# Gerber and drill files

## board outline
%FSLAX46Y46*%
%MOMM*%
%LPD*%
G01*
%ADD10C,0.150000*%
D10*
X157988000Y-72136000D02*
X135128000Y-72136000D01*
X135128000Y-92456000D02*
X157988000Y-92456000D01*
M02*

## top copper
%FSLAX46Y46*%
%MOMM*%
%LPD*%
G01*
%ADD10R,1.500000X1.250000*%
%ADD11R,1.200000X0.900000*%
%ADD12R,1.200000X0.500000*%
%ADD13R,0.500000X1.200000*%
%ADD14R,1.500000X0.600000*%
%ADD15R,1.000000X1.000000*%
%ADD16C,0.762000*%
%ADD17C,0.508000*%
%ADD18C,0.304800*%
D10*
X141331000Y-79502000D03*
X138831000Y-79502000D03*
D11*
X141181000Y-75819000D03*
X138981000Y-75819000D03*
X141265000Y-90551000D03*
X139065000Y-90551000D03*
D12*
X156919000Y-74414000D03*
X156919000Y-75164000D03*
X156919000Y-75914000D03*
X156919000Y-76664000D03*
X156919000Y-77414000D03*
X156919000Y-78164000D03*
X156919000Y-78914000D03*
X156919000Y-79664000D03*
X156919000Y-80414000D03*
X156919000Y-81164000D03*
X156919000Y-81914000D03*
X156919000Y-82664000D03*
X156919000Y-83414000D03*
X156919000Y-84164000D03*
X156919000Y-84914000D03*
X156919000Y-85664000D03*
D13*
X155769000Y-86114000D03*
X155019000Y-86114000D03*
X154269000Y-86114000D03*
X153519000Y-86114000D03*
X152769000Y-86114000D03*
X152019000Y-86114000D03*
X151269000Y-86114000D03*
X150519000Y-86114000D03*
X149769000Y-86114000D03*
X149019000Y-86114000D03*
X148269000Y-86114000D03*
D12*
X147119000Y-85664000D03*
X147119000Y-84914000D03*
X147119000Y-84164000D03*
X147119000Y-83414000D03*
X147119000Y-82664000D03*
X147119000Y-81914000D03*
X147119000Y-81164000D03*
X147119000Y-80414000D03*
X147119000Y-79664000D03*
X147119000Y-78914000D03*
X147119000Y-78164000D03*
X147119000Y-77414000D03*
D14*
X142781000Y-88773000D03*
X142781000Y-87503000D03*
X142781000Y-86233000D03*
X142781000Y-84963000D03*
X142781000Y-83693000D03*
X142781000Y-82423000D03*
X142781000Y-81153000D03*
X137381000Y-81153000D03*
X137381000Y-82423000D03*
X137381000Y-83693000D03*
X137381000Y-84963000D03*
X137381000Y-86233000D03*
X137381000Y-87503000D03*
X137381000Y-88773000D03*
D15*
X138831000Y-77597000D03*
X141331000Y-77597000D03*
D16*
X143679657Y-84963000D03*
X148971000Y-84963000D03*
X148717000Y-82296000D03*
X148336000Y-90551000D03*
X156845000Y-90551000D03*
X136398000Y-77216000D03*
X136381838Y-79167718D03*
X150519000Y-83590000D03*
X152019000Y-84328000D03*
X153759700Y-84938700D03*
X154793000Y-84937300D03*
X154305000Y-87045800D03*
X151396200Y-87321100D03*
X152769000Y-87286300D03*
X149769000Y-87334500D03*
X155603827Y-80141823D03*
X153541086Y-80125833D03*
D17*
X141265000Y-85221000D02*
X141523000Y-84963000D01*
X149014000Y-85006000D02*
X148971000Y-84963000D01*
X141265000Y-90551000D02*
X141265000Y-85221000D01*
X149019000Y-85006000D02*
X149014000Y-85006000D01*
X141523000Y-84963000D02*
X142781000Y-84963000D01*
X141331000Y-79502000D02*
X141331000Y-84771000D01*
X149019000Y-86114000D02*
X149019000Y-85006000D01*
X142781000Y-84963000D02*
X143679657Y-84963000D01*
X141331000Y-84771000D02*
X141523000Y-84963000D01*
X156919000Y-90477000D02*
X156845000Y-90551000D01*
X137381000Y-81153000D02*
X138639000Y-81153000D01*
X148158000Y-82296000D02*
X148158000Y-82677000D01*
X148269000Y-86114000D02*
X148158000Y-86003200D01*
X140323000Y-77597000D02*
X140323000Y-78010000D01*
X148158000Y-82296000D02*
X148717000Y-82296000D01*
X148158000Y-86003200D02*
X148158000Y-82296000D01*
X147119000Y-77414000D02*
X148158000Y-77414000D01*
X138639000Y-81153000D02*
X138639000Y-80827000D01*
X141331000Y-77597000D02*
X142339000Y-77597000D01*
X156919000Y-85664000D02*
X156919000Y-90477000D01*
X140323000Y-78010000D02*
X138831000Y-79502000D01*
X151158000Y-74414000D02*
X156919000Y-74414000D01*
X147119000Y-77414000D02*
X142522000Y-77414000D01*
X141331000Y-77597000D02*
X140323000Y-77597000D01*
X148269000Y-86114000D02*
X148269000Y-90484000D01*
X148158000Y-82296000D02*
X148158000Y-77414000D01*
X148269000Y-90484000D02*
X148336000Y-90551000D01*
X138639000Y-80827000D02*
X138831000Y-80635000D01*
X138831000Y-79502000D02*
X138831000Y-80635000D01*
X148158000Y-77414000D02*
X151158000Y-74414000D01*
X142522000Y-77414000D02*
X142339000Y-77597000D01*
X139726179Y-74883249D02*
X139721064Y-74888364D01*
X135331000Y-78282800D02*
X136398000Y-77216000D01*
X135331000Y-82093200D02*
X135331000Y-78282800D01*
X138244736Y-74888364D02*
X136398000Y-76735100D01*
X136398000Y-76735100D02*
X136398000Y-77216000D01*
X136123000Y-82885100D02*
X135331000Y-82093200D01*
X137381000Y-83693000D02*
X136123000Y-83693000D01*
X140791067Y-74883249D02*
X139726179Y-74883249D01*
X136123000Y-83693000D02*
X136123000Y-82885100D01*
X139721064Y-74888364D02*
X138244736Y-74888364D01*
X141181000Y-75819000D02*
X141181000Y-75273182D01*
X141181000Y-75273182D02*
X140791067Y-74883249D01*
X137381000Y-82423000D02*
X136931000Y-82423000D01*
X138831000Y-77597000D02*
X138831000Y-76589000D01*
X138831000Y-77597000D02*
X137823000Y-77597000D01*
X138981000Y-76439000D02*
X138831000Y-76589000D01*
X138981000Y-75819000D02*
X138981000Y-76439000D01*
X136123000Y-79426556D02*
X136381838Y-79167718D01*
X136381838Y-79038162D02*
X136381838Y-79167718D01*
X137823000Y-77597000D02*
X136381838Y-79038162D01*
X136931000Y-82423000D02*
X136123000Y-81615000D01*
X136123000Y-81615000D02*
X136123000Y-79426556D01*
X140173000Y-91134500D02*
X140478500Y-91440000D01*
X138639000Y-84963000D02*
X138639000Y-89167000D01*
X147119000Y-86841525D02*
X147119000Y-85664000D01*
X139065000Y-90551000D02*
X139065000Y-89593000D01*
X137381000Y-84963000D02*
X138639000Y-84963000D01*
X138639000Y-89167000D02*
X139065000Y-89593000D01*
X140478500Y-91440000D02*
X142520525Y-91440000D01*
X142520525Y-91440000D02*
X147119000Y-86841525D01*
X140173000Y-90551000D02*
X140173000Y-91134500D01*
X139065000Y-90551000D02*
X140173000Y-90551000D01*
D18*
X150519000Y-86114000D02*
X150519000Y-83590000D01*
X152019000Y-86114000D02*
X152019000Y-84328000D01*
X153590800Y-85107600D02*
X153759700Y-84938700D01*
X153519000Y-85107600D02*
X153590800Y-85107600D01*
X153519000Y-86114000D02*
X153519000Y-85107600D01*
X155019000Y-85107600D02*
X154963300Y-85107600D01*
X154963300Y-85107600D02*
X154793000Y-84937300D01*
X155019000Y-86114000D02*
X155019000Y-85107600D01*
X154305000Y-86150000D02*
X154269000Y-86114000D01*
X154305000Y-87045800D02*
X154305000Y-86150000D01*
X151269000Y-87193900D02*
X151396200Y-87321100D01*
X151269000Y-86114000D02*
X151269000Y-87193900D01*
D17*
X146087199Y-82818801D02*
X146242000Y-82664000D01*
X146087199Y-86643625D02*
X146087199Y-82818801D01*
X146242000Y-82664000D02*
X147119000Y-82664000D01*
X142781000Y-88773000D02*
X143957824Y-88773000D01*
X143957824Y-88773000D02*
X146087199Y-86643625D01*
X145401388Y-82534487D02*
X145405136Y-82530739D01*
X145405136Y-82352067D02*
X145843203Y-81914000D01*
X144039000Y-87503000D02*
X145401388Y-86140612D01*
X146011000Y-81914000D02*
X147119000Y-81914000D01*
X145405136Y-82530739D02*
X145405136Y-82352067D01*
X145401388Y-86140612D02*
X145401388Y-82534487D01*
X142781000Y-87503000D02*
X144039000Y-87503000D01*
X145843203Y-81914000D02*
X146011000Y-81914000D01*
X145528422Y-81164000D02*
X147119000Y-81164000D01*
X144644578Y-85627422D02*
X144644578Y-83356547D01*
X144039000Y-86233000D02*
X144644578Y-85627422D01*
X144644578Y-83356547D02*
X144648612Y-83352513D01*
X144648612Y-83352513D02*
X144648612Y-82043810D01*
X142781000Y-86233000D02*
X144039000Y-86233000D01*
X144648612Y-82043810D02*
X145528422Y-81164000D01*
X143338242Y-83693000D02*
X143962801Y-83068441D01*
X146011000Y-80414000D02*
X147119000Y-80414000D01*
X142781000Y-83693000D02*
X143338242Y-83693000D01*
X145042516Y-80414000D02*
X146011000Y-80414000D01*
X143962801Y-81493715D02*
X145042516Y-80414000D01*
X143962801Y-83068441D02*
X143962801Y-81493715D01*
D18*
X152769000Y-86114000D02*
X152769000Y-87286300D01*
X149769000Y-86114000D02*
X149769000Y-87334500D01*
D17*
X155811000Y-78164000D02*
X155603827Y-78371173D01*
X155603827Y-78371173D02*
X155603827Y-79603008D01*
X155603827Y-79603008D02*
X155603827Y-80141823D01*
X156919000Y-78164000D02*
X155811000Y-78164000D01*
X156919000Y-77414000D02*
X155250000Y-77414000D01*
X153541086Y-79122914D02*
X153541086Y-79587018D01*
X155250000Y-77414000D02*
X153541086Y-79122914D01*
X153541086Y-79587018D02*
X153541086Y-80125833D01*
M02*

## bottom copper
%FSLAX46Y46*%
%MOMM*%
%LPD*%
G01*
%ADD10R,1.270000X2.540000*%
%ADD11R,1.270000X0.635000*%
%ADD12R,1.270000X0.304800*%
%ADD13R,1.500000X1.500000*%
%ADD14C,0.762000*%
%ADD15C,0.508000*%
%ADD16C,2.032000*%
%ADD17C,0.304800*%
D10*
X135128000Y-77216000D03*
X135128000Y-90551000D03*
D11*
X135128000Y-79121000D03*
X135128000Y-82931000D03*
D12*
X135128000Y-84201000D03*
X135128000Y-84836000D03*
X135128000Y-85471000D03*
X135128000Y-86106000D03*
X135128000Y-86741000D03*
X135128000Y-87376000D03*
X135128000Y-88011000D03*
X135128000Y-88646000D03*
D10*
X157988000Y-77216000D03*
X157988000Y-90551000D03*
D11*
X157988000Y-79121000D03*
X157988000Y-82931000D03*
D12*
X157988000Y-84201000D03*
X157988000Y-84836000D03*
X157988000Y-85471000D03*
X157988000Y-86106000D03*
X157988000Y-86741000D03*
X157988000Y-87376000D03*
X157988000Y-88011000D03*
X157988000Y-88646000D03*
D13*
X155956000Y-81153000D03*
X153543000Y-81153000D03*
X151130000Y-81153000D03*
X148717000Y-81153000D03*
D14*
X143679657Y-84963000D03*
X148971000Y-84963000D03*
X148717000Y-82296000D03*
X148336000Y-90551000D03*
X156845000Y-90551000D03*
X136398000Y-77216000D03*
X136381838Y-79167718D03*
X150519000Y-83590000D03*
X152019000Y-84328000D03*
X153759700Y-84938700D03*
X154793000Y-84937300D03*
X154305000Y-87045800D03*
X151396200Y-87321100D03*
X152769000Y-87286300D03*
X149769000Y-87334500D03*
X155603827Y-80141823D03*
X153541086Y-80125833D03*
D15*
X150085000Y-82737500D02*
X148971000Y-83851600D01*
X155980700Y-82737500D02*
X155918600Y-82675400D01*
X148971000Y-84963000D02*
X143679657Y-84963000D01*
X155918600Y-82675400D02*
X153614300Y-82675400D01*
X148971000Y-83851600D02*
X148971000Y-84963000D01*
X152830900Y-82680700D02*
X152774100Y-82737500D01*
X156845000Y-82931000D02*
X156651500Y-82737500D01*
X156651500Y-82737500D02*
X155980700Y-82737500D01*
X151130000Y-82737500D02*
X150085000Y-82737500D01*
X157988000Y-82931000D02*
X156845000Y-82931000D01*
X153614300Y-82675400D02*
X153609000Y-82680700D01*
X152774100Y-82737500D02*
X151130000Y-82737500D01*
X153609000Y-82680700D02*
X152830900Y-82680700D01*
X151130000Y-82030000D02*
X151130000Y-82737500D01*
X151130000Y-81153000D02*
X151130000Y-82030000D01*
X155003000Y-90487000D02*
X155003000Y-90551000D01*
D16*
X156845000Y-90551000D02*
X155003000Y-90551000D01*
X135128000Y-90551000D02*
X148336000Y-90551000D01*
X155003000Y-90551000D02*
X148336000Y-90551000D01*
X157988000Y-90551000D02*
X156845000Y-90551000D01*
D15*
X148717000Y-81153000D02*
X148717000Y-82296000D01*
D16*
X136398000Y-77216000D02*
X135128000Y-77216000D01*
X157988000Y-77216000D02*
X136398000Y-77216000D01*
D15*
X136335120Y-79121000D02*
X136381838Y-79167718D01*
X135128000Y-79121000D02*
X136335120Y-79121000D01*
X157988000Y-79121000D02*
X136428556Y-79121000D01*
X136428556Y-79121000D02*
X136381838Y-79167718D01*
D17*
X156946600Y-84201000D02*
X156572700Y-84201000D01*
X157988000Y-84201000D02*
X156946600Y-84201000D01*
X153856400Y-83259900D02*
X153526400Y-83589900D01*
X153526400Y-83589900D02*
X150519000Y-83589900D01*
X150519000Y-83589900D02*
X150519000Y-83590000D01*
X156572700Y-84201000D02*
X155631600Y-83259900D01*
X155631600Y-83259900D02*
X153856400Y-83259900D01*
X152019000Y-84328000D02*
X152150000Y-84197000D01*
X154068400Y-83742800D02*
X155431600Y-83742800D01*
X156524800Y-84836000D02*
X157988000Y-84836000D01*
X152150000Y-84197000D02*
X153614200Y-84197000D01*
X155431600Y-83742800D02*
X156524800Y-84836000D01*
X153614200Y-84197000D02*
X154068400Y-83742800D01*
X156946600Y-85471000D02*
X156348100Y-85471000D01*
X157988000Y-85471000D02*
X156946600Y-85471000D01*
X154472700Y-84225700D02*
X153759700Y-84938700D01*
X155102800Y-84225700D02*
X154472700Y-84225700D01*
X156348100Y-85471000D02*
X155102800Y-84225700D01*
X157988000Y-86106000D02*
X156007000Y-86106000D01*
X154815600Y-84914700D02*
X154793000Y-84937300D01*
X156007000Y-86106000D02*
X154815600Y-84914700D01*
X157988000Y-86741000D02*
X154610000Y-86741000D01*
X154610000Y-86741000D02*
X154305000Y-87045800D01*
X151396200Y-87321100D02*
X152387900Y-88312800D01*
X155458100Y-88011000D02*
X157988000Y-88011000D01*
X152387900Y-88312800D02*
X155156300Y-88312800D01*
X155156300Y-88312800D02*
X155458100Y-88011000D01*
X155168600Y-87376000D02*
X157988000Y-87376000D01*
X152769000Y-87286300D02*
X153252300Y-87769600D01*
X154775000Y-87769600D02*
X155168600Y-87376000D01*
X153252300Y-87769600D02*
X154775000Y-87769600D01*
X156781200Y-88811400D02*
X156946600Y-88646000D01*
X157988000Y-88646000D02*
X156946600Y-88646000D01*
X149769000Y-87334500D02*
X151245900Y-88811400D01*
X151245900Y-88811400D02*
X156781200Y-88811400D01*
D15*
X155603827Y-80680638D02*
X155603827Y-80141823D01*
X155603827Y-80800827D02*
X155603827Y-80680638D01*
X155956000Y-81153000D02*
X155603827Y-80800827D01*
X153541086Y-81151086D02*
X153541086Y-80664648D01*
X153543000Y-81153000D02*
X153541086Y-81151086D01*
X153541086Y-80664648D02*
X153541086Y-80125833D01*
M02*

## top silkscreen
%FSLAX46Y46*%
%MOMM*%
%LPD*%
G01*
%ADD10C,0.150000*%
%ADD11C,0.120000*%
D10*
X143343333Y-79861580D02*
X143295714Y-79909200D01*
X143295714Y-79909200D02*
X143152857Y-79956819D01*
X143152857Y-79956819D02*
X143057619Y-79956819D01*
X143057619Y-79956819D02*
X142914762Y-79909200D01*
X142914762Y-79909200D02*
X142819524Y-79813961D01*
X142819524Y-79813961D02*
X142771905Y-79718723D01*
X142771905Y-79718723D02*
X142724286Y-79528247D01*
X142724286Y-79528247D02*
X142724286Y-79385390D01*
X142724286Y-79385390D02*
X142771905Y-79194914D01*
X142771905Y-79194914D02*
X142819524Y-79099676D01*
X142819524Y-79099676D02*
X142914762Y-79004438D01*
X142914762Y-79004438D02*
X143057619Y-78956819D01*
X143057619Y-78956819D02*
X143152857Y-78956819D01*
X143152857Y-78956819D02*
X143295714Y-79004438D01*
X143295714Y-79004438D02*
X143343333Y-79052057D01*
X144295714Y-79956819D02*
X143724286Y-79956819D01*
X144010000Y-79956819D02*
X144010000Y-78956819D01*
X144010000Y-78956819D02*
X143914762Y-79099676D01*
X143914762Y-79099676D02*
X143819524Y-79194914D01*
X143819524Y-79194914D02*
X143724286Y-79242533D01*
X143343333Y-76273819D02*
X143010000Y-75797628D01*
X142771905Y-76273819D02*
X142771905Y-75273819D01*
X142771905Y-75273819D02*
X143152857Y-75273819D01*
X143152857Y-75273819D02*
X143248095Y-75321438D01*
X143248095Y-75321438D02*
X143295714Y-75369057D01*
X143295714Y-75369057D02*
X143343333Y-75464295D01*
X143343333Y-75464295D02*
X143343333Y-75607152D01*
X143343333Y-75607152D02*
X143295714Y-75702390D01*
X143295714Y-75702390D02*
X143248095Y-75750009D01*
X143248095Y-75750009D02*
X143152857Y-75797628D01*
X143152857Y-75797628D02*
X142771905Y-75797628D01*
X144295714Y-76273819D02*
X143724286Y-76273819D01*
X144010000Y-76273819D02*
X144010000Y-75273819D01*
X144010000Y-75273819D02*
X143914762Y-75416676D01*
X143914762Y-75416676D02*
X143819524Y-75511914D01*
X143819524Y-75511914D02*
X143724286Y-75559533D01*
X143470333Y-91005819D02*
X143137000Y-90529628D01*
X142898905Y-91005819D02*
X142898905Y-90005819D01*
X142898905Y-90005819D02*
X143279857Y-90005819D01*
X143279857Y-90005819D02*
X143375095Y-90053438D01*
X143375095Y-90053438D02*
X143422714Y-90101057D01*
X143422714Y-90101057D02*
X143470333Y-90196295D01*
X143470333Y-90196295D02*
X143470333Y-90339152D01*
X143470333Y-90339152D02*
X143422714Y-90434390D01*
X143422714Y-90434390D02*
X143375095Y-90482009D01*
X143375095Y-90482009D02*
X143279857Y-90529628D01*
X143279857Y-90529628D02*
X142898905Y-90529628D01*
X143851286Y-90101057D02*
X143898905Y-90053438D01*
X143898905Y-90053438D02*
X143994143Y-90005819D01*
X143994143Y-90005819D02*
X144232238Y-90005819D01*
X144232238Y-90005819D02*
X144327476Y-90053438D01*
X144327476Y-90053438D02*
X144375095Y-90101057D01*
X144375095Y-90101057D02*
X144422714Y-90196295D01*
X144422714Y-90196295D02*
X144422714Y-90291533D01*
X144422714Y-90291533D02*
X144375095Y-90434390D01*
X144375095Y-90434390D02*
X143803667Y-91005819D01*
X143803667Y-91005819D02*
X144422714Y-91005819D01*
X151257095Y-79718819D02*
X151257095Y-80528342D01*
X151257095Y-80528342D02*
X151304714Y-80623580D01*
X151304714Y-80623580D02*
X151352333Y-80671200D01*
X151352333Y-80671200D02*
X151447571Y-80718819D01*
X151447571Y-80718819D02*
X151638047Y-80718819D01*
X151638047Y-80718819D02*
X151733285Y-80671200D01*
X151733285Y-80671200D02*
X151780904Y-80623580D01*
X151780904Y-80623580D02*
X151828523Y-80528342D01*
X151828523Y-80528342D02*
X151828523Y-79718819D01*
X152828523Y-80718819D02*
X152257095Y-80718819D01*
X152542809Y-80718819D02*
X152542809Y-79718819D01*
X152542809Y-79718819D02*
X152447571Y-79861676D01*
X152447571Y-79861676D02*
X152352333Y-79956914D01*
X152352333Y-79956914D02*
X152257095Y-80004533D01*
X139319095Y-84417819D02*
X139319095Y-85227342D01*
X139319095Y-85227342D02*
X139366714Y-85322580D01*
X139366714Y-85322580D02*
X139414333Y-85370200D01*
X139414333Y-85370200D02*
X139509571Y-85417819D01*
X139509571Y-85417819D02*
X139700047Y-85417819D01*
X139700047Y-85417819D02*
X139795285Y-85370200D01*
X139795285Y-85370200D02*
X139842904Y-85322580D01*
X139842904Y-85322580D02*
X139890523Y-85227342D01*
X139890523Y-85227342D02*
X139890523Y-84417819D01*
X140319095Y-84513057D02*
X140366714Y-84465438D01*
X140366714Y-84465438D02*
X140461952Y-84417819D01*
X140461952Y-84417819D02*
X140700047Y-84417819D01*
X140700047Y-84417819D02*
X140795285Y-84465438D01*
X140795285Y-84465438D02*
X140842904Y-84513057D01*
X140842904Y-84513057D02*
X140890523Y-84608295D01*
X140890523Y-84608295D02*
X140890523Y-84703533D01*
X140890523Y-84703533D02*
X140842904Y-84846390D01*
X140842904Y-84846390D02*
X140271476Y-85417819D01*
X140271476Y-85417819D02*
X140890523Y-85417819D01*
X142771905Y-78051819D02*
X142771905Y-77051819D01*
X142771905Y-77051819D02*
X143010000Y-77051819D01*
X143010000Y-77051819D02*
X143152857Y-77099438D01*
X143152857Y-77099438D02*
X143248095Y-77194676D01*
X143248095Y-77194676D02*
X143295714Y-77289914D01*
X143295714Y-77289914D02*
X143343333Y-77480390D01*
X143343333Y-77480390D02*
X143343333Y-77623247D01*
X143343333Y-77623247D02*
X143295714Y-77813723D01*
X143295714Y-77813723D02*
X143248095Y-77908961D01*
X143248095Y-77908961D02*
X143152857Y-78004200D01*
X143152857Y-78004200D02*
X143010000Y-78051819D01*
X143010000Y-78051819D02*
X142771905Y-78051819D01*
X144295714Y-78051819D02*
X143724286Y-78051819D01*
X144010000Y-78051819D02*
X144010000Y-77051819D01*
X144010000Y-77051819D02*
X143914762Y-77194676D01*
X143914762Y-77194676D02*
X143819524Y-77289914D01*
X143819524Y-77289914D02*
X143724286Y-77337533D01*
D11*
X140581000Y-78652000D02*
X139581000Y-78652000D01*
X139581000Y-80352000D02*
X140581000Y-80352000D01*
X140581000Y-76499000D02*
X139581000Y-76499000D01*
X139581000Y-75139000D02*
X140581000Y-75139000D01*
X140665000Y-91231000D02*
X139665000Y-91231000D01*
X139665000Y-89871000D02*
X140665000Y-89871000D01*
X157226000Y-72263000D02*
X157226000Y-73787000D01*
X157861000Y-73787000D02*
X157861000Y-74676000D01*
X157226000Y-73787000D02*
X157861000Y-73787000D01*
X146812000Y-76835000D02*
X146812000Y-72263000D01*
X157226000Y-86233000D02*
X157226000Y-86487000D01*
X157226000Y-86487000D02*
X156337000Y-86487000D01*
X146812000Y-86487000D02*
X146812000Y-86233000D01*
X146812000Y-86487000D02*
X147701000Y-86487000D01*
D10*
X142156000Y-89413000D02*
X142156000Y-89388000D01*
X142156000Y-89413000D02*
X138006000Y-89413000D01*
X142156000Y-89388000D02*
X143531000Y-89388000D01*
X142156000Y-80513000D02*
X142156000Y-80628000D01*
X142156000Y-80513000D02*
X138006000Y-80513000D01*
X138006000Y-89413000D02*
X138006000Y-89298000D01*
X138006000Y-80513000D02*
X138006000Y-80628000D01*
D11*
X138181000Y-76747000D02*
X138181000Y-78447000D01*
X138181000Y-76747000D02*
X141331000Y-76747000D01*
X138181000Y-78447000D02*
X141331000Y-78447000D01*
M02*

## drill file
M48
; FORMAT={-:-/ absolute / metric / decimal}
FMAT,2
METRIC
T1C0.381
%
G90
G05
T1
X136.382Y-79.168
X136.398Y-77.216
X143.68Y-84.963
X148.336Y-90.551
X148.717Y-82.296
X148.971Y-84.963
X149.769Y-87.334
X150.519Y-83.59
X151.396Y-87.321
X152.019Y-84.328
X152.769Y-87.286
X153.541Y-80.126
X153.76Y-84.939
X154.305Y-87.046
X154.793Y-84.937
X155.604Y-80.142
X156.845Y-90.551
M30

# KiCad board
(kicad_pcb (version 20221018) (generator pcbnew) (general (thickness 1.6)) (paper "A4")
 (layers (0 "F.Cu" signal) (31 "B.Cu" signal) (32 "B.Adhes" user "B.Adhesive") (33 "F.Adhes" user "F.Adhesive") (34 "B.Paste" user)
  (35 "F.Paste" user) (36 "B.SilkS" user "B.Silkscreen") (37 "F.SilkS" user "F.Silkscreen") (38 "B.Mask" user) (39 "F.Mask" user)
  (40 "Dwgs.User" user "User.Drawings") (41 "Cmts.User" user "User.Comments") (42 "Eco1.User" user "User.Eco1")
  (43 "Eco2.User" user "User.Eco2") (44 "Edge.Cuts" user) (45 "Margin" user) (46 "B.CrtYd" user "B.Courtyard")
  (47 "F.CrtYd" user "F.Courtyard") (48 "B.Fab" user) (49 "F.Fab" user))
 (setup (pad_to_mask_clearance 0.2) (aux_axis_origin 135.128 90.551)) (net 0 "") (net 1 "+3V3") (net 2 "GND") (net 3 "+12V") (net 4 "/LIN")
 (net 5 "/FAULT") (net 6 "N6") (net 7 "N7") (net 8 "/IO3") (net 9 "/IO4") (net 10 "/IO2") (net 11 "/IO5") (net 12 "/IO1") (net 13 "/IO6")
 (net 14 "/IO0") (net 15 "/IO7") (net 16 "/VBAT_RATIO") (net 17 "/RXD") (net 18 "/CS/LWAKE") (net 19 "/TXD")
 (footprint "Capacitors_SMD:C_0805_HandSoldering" (layer "F.Cu") (at 140.081 79.502 180)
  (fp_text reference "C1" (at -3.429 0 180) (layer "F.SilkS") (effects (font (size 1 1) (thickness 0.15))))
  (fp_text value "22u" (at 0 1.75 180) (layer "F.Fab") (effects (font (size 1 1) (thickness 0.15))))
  (fp_line (start -0.5 0.85) (end 0.5 0.85) (stroke (width 0.12) (type solid)) (layer "F.SilkS"))
  (fp_line (start 0.5 -0.85) (end -0.5 -0.85) (stroke (width 0.12) (type solid)) (layer "F.SilkS"))
  (pad "1" smd rect (at -1.25 0 180) (size 1.5 1.25) (layers "F.Cu" "F.Paste" "F.Mask") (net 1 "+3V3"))
  (pad "2" smd rect (at 1.25 0 180) (size 1.5 1.25) (layers "F.Cu" "F.Paste" "F.Mask") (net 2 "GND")))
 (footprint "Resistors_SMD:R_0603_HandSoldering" (layer "F.Cu") (at 140.081 75.819 180)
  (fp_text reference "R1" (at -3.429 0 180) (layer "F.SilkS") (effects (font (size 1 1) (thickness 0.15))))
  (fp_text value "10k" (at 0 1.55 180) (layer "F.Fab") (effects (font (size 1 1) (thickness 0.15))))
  (fp_line (start -0.5 -0.68) (end 0.5 -0.68) (stroke (width 0.12) (type solid)) (layer "F.SilkS"))
  (fp_line (start 0.5 0.68) (end -0.5 0.68) (stroke (width 0.12) (type solid)) (layer "F.SilkS"))
  (pad "1" smd rect (at -1.1 0 180) (size 1.2 0.9) (layers "F.Cu" "F.Paste" "F.Mask") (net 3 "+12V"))
  (pad "2" smd rect (at 1.1 0 180) (size 1.2 0.9) (layers "F.Cu" "F.Paste" "F.Mask") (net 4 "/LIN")))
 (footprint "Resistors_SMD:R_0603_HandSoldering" (layer "F.Cu") (at 140.165 90.551 180)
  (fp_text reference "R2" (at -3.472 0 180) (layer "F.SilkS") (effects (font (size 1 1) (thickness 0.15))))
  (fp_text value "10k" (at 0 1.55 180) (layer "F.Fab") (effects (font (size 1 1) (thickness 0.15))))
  (fp_line (start -0.5 -0.68) (end 0.5 -0.68) (stroke (width 0.12) (type solid)) (layer "F.SilkS"))
  (fp_line (start 0.5 0.68) (end -0.5 0.68) (stroke (width 0.12) (type solid)) (layer "F.SilkS"))
  (pad "1" smd rect (at -1.1 0 180) (size 1.2 0.9) (layers "F.Cu" "F.Paste" "F.Mask") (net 1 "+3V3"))
  (pad "2" smd rect (at 1.1 0 180) (size 1.2 0.9) (layers "F.Cu" "F.Paste" "F.Mask") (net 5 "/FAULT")))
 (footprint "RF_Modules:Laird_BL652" (layer "F.Cu") (at 152.019 80.264 -90)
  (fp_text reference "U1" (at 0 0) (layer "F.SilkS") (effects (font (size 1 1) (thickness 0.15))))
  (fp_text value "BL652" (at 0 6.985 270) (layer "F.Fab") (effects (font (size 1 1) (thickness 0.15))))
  (fp_line (start -8.001 -5.207) (end -6.477 -5.207) (stroke (width 0.12) (type solid)) (layer "F.SilkS"))
  (fp_line (start -6.477 -5.842) (end -5.588 -5.842) (stroke (width 0.12) (type solid)) (layer "F.SilkS"))
  (fp_line (start -6.477 -5.207) (end -6.477 -5.842) (stroke (width 0.12) (type solid)) (layer "F.SilkS"))
  (fp_line (start -3.429 5.207) (end -8.001 5.207) (stroke (width 0.12) (type solid)) (layer "F.SilkS"))
  (fp_line (start 5.969 -5.207) (end 6.223 -5.207) (stroke (width 0.12) (type solid)) (layer "F.SilkS"))
  (fp_line (start 6.223 -5.207) (end 6.223 -4.318) (stroke (width 0.12) (type solid)) (layer "F.SilkS"))
  (fp_line (start 6.223 5.207) (end 5.969 5.207) (stroke (width 0.12) (type solid)) (layer "F.SilkS"))
  (fp_line (start 6.223 5.207) (end 6.223 4.318) (stroke (width 0.12) (type solid)) (layer "F.SilkS"))
  (pad "1" smd rect (at -5.85 -4.9) (size 1.2 0.5) (layers "F.Cu" "F.Paste" "F.Mask") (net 2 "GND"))
  (pad "2" smd rect (at -5.1 -4.9) (size 1.2 0.5) (layers "F.Cu" "F.Paste" "F.Mask"))
  (pad "3" smd rect (at -4.35 -4.9) (size 1.2 0.5) (layers "F.Cu" "F.Paste" "F.Mask"))
  (pad "4" smd rect (at -3.6 -4.9) (size 1.2 0.5) (layers "F.Cu" "F.Paste" "F.Mask"))
  (pad "5" smd rect (at -2.85 -4.9) (size 1.2 0.5) (layers "F.Cu" "F.Paste" "F.Mask") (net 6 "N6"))
  (pad "6" smd rect (at -2.1 -4.9) (size 1.2 0.5) (layers "F.Cu" "F.Paste" "F.Mask") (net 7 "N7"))
  (pad "7" smd rect (at -1.35 -4.9) (size 1.2 0.5) (layers "F.Cu" "F.Paste" "F.Mask"))
  (pad "8" smd rect (at -0.6 -4.9) (size 1.2 0.5) (layers "F.Cu" "F.Paste" "F.Mask"))
  (pad "9" smd rect (at 0.15 -4.9) (size 1.2 0.5) (layers "F.Cu" "F.Paste" "F.Mask"))
  (pad "10" smd rect (at 0.9 -4.9) (size 1.2 0.5) (layers "F.Cu" "F.Paste" "F.Mask"))
  (pad "11" smd rect (at 1.65 -4.9) (size 1.2 0.5) (layers "F.Cu" "F.Paste" "F.Mask"))
  (pad "12" smd rect (at 2.4 -4.9) (size 1.2 0.5) (layers "F.Cu" "F.Paste" "F.Mask"))
  (pad "13" smd rect (at 3.15 -4.9) (size 1.2 0.5) (layers "F.Cu" "F.Paste" "F.Mask"))
  (pad "14" smd rect (at 3.9 -4.9) (size 1.2 0.5) (layers "F.Cu" "F.Paste" "F.Mask"))
  (pad "15" smd rect (at 4.65 -4.9) (size 1.2 0.5) (layers "F.Cu" "F.Paste" "F.Mask"))
  (pad "16" smd rect (at 5.4 -4.9) (size 1.2 0.5) (layers "F.Cu" "F.Paste" "F.Mask") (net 2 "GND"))
  (pad "17" smd rect (at 5.85 -3.75 270) (size 1.2 0.5) (layers "F.Cu" "F.Paste" "F.Mask"))
  (pad "18" smd rect (at 5.85 -3 270) (size 1.2 0.5) (layers "F.Cu" "F.Paste" "F.Mask") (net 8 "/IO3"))
  (pad "19" smd rect (at 5.85 -2.25 270) (size 1.2 0.5) (layers "F.Cu" "F.Paste" "F.Mask") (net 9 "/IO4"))
  (pad "20" smd rect (at 5.85 -1.5 270) (size 1.2 0.5) (layers "F.Cu" "F.Paste" "F.Mask") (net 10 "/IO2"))
  (pad "21" smd rect (at 5.85 -0.75 270) (size 1.2 0.5) (layers "F.Cu" "F.Paste" "F.Mask") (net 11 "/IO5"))
  (pad "22" smd rect (at 5.85 0 270) (size 1.2 0.5) (layers "F.Cu" "F.Paste" "F.Mask") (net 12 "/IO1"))
  (pad "23" smd rect (at 5.85 0.75 270) (size 1.2 0.5) (layers "F.Cu" "F.Paste" "F.Mask") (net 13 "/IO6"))
  (pad "24" smd rect (at 5.85 1.5 270) (size 1.2 0.5) (layers "F.Cu" "F.Paste" "F.Mask") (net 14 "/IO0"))
  (pad "25" smd rect (at 5.85 2.25 270) (size 1.2 0.5) (layers "F.Cu" "F.Paste" "F.Mask") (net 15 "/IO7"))
  (pad "26" smd rect (at 5.85 3 270) (size 1.2 0.5) (layers "F.Cu" "F.Paste" "F.Mask") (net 1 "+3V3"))
  (pad "27" smd rect (at 5.85 3.75 270) (size 1.2 0.5) (layers "F.Cu" "F.Paste" "F.Mask") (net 2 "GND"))
  (pad "28" smd rect (at 5.4 4.9) (size 1.2 0.5) (layers "F.Cu" "F.Paste" "F.Mask") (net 5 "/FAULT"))
  (pad "29" smd rect (at 4.65 4.9) (size 1.2 0.5) (layers "F.Cu" "F.Paste" "F.Mask"))
  (pad "30" smd rect (at 3.9 4.9) (size 1.2 0.5) (layers "F.Cu" "F.Paste" "F.Mask"))
  (pad "31" smd rect (at 3.15 4.9) (size 1.2 0.5) (layers "F.Cu" "F.Paste" "F.Mask"))
  (pad "32" smd rect (at 2.4 4.9) (size 1.2 0.5) (layers "F.Cu" "F.Paste" "F.Mask") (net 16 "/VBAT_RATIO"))
  (pad "33" smd rect (at 1.65 4.9) (size 1.2 0.5) (layers "F.Cu" "F.Paste" "F.Mask") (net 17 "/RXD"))
  (pad "34" smd rect (at 0.9 4.9) (size 1.2 0.5) (layers "F.Cu" "F.Paste" "F.Mask") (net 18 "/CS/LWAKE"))
  (pad "35" smd rect (at 0.15 4.9) (size 1.2 0.5) (layers "F.Cu" "F.Paste" "F.Mask") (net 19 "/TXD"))
  (pad "36" smd rect (at -0.6 4.9) (size 1.2 0.5) (layers "F.Cu" "F.Paste" "F.Mask"))
  (pad "37" smd rect (at -1.35 4.9) (size 1.2 0.5) (layers "F.Cu" "F.Paste" "F.Mask"))
  (pad "38" smd rect (at -2.1 4.9) (size 1.2 0.5) (layers "F.Cu" "F.Paste" "F.Mask"))
  (pad "39" smd rect (at -2.85 4.9) (size 1.2 0.5) (layers "F.Cu" "F.Paste" "F.Mask") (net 2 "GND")))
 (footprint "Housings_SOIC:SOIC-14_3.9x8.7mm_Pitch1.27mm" (layer "F.Cu") (at 140.081 84.963 180)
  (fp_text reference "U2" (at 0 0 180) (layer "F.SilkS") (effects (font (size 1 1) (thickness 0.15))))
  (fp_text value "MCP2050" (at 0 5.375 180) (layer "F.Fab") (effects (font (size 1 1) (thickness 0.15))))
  (fp_line (start -2.075 -4.45) (end -2.075 -4.425) (stroke (width 0.15) (type solid)) (layer "F.SilkS"))
  (fp_line (start -2.075 -4.45) (end 2.075 -4.45) (stroke (width 0.15) (type solid)) (layer "F.SilkS"))
  (fp_line (start -2.075 -4.425) (end -3.45 -4.425) (stroke (width 0.15) (type solid)) (layer "F.SilkS"))
  (fp_line (start -2.075 4.45) (end -2.075 4.335) (stroke (width 0.15) (type solid)) (layer "F.SilkS"))
  (fp_line (start -2.075 4.45) (end 2.075 4.45) (stroke (width 0.15) (type solid)) (layer "F.SilkS"))
  (fp_line (start 2.075 -4.45) (end 2.075 -4.335) (stroke (width 0.15) (type solid)) (layer "F.SilkS"))
  (fp_line (start 2.075 4.45) (end 2.075 4.335) (stroke (width 0.15) (type solid)) (layer "F.SilkS"))
  (pad "1" smd rect (at -2.7 -3.81 180) (size 1.5 0.6) (layers "F.Cu" "F.Paste" "F.Mask") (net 16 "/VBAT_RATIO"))
  (pad "2" smd rect (at -2.7 -2.54 180) (size 1.5 0.6) (layers "F.Cu" "F.Paste" "F.Mask") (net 17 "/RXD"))
  (pad "3" smd rect (at -2.7 -1.27 180) (size 1.5 0.6) (layers "F.Cu" "F.Paste" "F.Mask") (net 18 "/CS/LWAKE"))
  (pad "4" smd rect (at -2.7 0 180) (size 1.5 0.6) (layers "F.Cu" "F.Paste" "F.Mask") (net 1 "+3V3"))
  (pad "5" smd rect (at -2.7 1.27 180) (size 1.5 0.6) (layers "F.Cu" "F.Paste" "F.Mask") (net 19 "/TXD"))
  (pad "6" smd rect (at -2.7 2.54 180) (size 1.5 0.6) (layers "F.Cu" "F.Paste" "F.Mask"))
  (pad "7" smd rect (at -2.7 3.81 180) (size 1.5 0.6) (layers "F.Cu" "F.Paste" "F.Mask"))
  (pad "8" smd rect (at 2.7 3.81 180) (size 1.5 0.6) (layers "F.Cu" "F.Paste" "F.Mask") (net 2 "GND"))
  (pad "9" smd rect (at 2.7 2.54 180) (size 1.5 0.6) (layers "F.Cu" "F.Paste" "F.Mask") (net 4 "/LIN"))
  (pad "10" smd rect (at 2.7 1.27 180) (size 1.5 0.6) (layers "F.Cu" "F.Paste" "F.Mask") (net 3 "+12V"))
  (pad "11" smd rect (at 2.7 0 180) (size 1.5 0.6) (layers "F.Cu" "F.Paste" "F.Mask") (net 5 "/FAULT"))
  (pad "12" smd rect (at 2.7 -1.27 180) (size 1.5 0.6) (layers "F.Cu" "F.Paste" "F.Mask"))
  (pad "13" smd rect (at 2.7 -2.54 180) (size 1.5 0.6) (layers "F.Cu" "F.Paste" "F.Mask"))
  (pad "14" smd rect (at 2.7 -3.81 180) (size 1.5 0.6) (layers "F.Cu" "F.Paste" "F.Mask")))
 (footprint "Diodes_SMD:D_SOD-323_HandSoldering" (layer "F.Cu") (at 140.081 77.597)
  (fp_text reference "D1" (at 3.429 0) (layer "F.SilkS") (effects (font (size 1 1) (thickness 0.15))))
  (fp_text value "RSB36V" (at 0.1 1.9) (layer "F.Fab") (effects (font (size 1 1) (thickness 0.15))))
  (fp_line (start -1.9 -0.85) (end -1.9 0.85) (stroke (width 0.12) (type solid)) (layer "F.SilkS"))
  (fp_line (start -1.9 -0.85) (end 1.25 -0.85) (stroke (width 0.12) (type solid)) (layer "F.SilkS"))
  (fp_line (start -1.9 0.85) (end 1.25 0.85) (stroke (width 0.12) (type solid)) (layer "F.SilkS"))
  (pad "1" smd rect (at -1.25 0) (size 1 1) (layers "F.Cu" "F.Paste" "F.Mask") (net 4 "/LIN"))
  (pad "2" smd rect (at 1.25 0) (size 1 1) (layers "F.Cu" "F.Paste" "F.Mask") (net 2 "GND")))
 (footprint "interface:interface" (layer "F.Cu") (at 135.128 72.771)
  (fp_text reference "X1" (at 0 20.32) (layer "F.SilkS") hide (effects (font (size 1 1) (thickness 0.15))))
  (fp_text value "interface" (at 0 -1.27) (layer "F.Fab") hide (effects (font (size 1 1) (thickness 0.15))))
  (pad "1" smd rect (at 0 4.445) (size 1.27 2.54) (layers "B.Cu") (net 3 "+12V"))
  (pad "2" smd rect (at 0 17.78) (size 1.27 2.54) (layers "B.Cu") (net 2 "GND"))
  (pad "3" smd rect (at 0 6.35) (size 1.27 0.635) (layers "B.Cu") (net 4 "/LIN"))
  (pad "4" smd rect (at 0 10.16) (size 1.27 0.635) (layers "B.Cu"))
  (pad "5" smd rect (at 0 11.43) (size 1.27 0.3048) (layers "B.Cu"))
  (pad "6" smd rect (at 0 12.065) (size 1.27 0.3048) (layers "B.Cu"))
  (pad "7" smd rect (at 0 12.7) (size 1.27 0.3048) (layers "B.Cu"))
  (pad "8" smd rect (at 0 13.335) (size 1.27 0.3048) (layers "B.Cu"))
  (pad "9" smd rect (at 0 13.97) (size 1.27 0.3048) (layers "B.Cu"))
  (pad "10" smd rect (at 0 14.605) (size 1.27 0.3048) (layers "B.Cu"))
  (pad "11" smd rect (at 0 15.24) (size 1.27 0.3048) (layers "B.Cu"))
  (pad "12" smd rect (at 0 15.875) (size 1.27 0.3048) (layers "B.Cu")))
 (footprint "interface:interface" (layer "F.Cu") (at 157.988 72.771)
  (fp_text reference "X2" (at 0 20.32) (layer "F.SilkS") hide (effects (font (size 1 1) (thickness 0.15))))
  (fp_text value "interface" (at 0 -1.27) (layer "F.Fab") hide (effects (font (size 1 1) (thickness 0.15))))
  (pad "1" smd rect (at 0 4.445) (size 1.27 2.54) (layers "B.Cu") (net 3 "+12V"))
  (pad "2" smd rect (at 0 17.78) (size 1.27 2.54) (layers "B.Cu") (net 2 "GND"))
  (pad "3" smd rect (at 0 6.35) (size 1.27 0.635) (layers "B.Cu") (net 4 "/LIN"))
  (pad "4" smd rect (at 0 10.16) (size 1.27 0.635) (layers "B.Cu") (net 1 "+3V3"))
  (pad "5" smd rect (at 0 11.43) (size 1.27 0.3048) (layers "B.Cu") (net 14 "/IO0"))
  (pad "6" smd rect (at 0 12.065) (size 1.27 0.3048) (layers "B.Cu") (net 12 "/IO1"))
  (pad "7" smd rect (at 0 12.7) (size 1.27 0.3048) (layers "B.Cu") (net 10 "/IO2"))
  (pad "8" smd rect (at 0 13.335) (size 1.27 0.3048) (layers "B.Cu") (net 8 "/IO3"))
  (pad "9" smd rect (at 0 13.97) (size 1.27 0.3048) (layers "B.Cu") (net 9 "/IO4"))
  (pad "10" smd rect (at 0 14.605) (size 1.27 0.3048) (layers "B.Cu") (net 11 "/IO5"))
  (pad "11" smd rect (at 0 15.24) (size 1.27 0.3048) (layers "B.Cu") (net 13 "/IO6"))
  (pad "12" smd rect (at 0 15.875) (size 1.27 0.3048) (layers "B.Cu") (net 15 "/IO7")))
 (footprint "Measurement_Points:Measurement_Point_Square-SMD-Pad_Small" (layer "B.Cu") (at 155.956 81.153)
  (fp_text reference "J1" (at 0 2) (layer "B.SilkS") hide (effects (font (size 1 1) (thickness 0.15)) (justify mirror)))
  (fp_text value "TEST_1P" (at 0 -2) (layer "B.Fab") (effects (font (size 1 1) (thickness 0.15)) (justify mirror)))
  (pad "1" smd rect (at 0 0) (size 1.5 1.5) (layers "B.Cu" "B.Mask") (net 7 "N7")))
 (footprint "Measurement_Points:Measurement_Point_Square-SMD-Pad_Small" (layer "B.Cu") (at 153.543 81.153)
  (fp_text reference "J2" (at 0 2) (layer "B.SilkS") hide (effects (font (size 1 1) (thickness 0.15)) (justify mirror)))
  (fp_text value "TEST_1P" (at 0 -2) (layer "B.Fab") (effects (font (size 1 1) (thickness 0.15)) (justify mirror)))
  (pad "1" smd rect (at 0 0) (size 1.5 1.5) (layers "B.Cu" "B.Mask") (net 6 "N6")))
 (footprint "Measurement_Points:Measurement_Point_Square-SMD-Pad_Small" (layer "B.Cu") (at 151.13 81.153)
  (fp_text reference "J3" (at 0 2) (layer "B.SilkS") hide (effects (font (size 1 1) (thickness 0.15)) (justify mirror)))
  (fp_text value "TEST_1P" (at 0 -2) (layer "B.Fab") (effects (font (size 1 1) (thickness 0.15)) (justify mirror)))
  (pad "1" smd rect (at 0 0) (size 1.5 1.5) (layers "B.Cu" "B.Mask") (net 1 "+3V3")))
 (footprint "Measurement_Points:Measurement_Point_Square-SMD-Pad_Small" (layer "B.Cu") (at 148.717 81.153)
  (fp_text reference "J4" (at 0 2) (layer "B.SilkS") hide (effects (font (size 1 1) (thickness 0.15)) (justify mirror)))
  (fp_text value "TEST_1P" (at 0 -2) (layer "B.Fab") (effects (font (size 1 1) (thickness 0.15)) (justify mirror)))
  (pad "1" smd rect (at 0 0) (size 1.5 1.5) (layers "B.Cu" "B.Mask") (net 2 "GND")))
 (gr_line (start 157.988 72.136) (end 135.128 72.136) (stroke (width 0.15) (type solid)) (layer "Edge.Cuts"))
 (gr_line (start 135.128 92.456) (end 157.988 92.456) (stroke (width 0.15) (type solid)) (layer "Edge.Cuts"))
 (segment (start 141.265 85.221) (end 141.523 84.963) (width 0.508) (layer "F.Cu") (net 1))
 (segment (start 149.014 85.006) (end 148.971 84.963) (width 0.508) (layer "F.Cu") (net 1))
 (segment (start 141.265 90.551) (end 141.265 85.221) (width 0.508) (layer "F.Cu") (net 1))
 (segment (start 149.019 85.006) (end 149.014 85.006) (width 0.508) (layer "F.Cu") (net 1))
 (segment (start 141.523 84.963) (end 142.781 84.963) (width 0.508) (layer "F.Cu") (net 1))
 (segment (start 141.331 79.502) (end 141.331 84.771) (width 0.508) (layer "F.Cu") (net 1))
 (segment (start 149.019 86.114) (end 149.019 85.006) (width 0.508) (layer "F.Cu") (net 1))
 (segment (start 142.781 84.963) (end 143.679657 84.963) (width 0.508) (layer "F.Cu") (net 1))
 (segment (start 141.331 84.771) (end 141.523 84.963) (width 0.508) (layer "F.Cu") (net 1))
 (via (at 143.679657 84.963) (size 0.762) (drill 0.381) (layers "F.Cu" "B.Cu") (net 1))
 (via (at 148.971 84.963) (size 0.762) (drill 0.381) (layers "F.Cu" "B.Cu") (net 1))
 (segment (start 150.085 82.7375) (end 148.971 83.8516) (width 0.508) (layer "B.Cu") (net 1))
 (segment (start 155.9807 82.7375) (end 155.9186 82.6754) (width 0.508) (layer "B.Cu") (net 1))
 (segment (start 148.971 84.963) (end 143.679657 84.963) (width 0.508) (layer "B.Cu") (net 1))
 (segment (start 155.9186 82.6754) (end 153.6143 82.6754) (width 0.508) (layer "B.Cu") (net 1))
 (segment (start 148.971 83.8516) (end 148.971 84.963) (width 0.508) (layer "B.Cu") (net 1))
 (segment (start 152.8309 82.6807) (end 152.7741 82.7375) (width 0.508) (layer "B.Cu") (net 1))
 (segment (start 156.845 82.931) (end 156.6515 82.7375) (width 0.508) (layer "B.Cu") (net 1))
 (segment (start 156.6515 82.7375) (end 155.9807 82.7375) (width 0.508) (layer "B.Cu") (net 1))
 (segment (start 151.13 82.7375) (end 150.085 82.7375) (width 0.508) (layer "B.Cu") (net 1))
 (segment (start 157.988 82.931) (end 156.845 82.931) (width 0.508) (layer "B.Cu") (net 1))
 (segment (start 153.6143 82.6754) (end 153.609 82.6807) (width 0.508) (layer "B.Cu") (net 1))
 (segment (start 152.7741 82.7375) (end 151.13 82.7375) (width 0.508) (layer "B.Cu") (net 1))
 (segment (start 153.609 82.6807) (end 152.8309 82.6807) (width 0.508) (layer "B.Cu") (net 1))
 (segment (start 151.13 82.03) (end 151.13 82.7375) (width 0.508) (layer "B.Cu") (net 1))
 (segment (start 151.13 81.153) (end 151.13 82.03) (width 0.508) (layer "B.Cu") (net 1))
 (segment (start 156.919 90.477) (end 156.845 90.551) (width 0.508) (layer "F.Cu") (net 2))
 (segment (start 137.381 81.153) (end 138.639 81.153) (width 0.508) (layer "F.Cu") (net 2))
 (segment (start 148.158 82.296) (end 148.158 82.677) (width 0.508) (layer "F.Cu") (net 2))
 (segment (start 148.269 86.114) (end 148.158 86.0032) (width 0.508) (layer "F.Cu") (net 2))
 (segment (start 140.323 77.597) (end 140.323 78.01) (width 0.508) (layer "F.Cu") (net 2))
 (segment (start 148.158 82.296) (end 148.717 82.296) (width 0.508) (layer "F.Cu") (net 2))
 (segment (start 148.158 86.0032) (end 148.158 82.296) (width 0.508) (layer "F.Cu") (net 2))
 (segment (start 147.119 77.414) (end 148.158 77.414) (width 0.508) (layer "F.Cu") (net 2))
 (segment (start 138.639 81.153) (end 138.639 80.827) (width 0.508) (layer "F.Cu") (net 2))
 (segment (start 141.331 77.597) (end 142.339 77.597) (width 0.508) (layer "F.Cu") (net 2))
 (segment (start 156.919 85.664) (end 156.919 90.477) (width 0.508) (layer "F.Cu") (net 2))
 (segment (start 140.323 78.01) (end 138.831 79.502) (width 0.508) (layer "F.Cu") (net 2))
 (segment (start 151.158 74.414) (end 156.919 74.414) (width 0.508) (layer "F.Cu") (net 2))
 (segment (start 147.119 77.414) (end 142.522 77.414) (width 0.508) (layer "F.Cu") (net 2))
 (segment (start 141.331 77.597) (end 140.323 77.597) (width 0.508) (layer "F.Cu") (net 2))
 (segment (start 148.269 86.114) (end 148.269 90.484) (width 0.508) (layer "F.Cu") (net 2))
 (segment (start 148.158 82.296) (end 148.158 77.414) (width 0.508) (layer "F.Cu") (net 2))
 (segment (start 148.269 90.484) (end 148.336 90.551) (width 0.508) (layer "F.Cu") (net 2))
 (segment (start 138.639 80.827) (end 138.831 80.635) (width 0.508) (layer "F.Cu") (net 2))
 (segment (start 138.831 79.502) (end 138.831 80.635) (width 0.508) (layer "F.Cu") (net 2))
 (segment (start 148.158 77.414) (end 151.158 74.414) (width 0.508) (layer "F.Cu") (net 2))
 (segment (start 142.522 77.414) (end 142.339 77.597) (width 0.508) (layer "F.Cu") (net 2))
 (via (at 148.717 82.296) (size 0.762) (drill 0.381) (layers "F.Cu" "B.Cu") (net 2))
 (via (at 148.336 90.551) (size 0.762) (drill 0.381) (layers "F.Cu" "B.Cu") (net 2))
 (via (at 156.845 90.551) (size 0.762) (drill 0.381) (layers "F.Cu" "B.Cu") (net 2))
 (segment (start 155.003 90.487) (end 155.003 90.551) (width 0.508) (layer "B.Cu") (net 2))
 (segment (start 156.845 90.551) (end 155.003 90.551) (width 2.032) (layer "B.Cu") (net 2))
 (segment (start 135.128 90.551) (end 148.336 90.551) (width 2.032) (layer "B.Cu") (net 2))
 (segment (start 155.003 90.551) (end 148.336 90.551) (width 2.032) (layer "B.Cu") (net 2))
 (segment (start 157.988 90.551) (end 156.845 90.551) (width 2.032) (layer "B.Cu") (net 2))
 (segment (start 148.717 81.153) (end 148.717 82.296) (width 0.508) (layer "B.Cu") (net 2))
 (segment (start 139.726179 74.883249) (end 139.721064 74.888364) (width 0.508) (layer "F.Cu") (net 3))
 (segment (start 135.331 78.2828) (end 136.398 77.216) (width 0.508) (layer "F.Cu") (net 3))
 (segment (start 135.331 82.0932) (end 135.331 78.2828) (width 0.508) (layer "F.Cu") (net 3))
 (segment (start 138.244736 74.888364) (end 136.398 76.7351) (width 0.508) (layer "F.Cu") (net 3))
 (segment (start 136.398 76.7351) (end 136.398 77.216) (width 0.508) (layer "F.Cu") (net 3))
 (segment (start 136.123 82.8851) (end 135.331 82.0932) (width 0.508) (layer "F.Cu") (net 3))
 (segment (start 137.381 83.693) (end 136.123 83.693) (width 0.508) (layer "F.Cu") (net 3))
 (segment (start 140.791067 74.883249) (end 139.726179 74.883249) (width 0.508) (layer "F.Cu") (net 3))
 (segment (start 136.123 83.693) (end 136.123 82.8851) (width 0.508) (layer "F.Cu") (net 3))
 (segment (start 139.721064 74.888364) (end 138.244736 74.888364) (width 0.508) (layer "F.Cu") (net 3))
 (segment (start 141.181 75.819) (end 141.181 75.273182) (width 0.508) (layer "F.Cu") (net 3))
 (segment (start 141.181 75.273182) (end 140.791067 74.883249) (width 0.508) (layer "F.Cu") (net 3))
 (via (at 136.398 77.216) (size 0.762) (drill 0.381) (layers "F.Cu" "B.Cu") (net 3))
 (segment (start 136.398 77.216) (end 135.128 77.216) (width 2.032) (layer "B.Cu") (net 3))
 (segment (start 157.988 77.216) (end 136.398 77.216) (width 2.032) (layer "B.Cu") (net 3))
 (segment (start 137.381 82.423) (end 136.931 82.423) (width 0.508) (layer "F.Cu") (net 4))
 (segment (start 138.831 77.597) (end 138.831 76.589) (width 0.508) (layer "F.Cu") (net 4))
 (segment (start 138.831 77.597) (end 137.823 77.597) (width 0.508) (layer "F.Cu") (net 4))
 (segment (start 138.981 76.439) (end 138.831 76.589) (width 0.508) (layer "F.Cu") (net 4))
 (segment (start 138.981 75.819) (end 138.981 76.439) (width 0.508) (layer "F.Cu") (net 4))
 (segment (start 136.123 79.426556) (end 136.381838 79.167718) (width 0.508) (layer "F.Cu") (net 4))
 (segment (start 136.381838 79.038162) (end 136.381838 79.167718) (width 0.508) (layer "F.Cu") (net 4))
 (segment (start 137.823 77.597) (end 136.381838 79.038162) (width 0.508) (layer "F.Cu") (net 4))
 (segment (start 136.931 82.423) (end 136.123 81.615) (width 0.508) (layer "F.Cu") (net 4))
 (segment (start 136.123 81.615) (end 136.123 79.426556) (width 0.508) (layer "F.Cu") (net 4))
 (via (at 136.381838 79.167718) (size 0.762) (drill 0.381) (layers "F.Cu" "B.Cu") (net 4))
 (segment (start 136.33512 79.121) (end 136.381838 79.167718) (width 0.508) (layer "B.Cu") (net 4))
 (segment (start 135.128 79.121) (end 136.33512 79.121) (width 0.508) (layer "B.Cu") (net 4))
 (segment (start 157.988 79.121) (end 136.428556 79.121) (width 0.508) (layer "B.Cu") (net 4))
 (segment (start 136.428556 79.121) (end 136.381838 79.167718) (width 0.508) (layer "B.Cu") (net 4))
 (segment (start 140.173 91.1345) (end 140.4785 91.44) (width 0.508) (layer "F.Cu") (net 5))
 (segment (start 138.639 84.963) (end 138.639 89.167) (width 0.508) (layer "F.Cu") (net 5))
 (segment (start 147.119 86.841525) (end 147.119 85.664) (width 0.508) (layer "F.Cu") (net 5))
 (segment (start 139.065 90.551) (end 139.065 89.593) (width 0.508) (layer "F.Cu") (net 5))
 (segment (start 137.381 84.963) (end 138.639 84.963) (width 0.508) (layer "F.Cu") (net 5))
 (segment (start 138.639 89.167) (end 139.065 89.593) (width 0.508) (layer "F.Cu") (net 5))
 (segment (start 140.4785 91.44) (end 142.520525 91.44) (width 0.508) (layer "F.Cu") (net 5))
 (segment (start 142.520525 91.44) (end 147.119 86.841525) (width 0.508) (layer "F.Cu") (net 5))
 (segment (start 140.173 90.551) (end 140.173 91.1345) (width 0.508) (layer "F.Cu") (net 5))
 (segment (start 139.065 90.551) (end 140.173 90.551) (width 0.508) (layer "F.Cu") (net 5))
 (segment (start 150.519 86.114) (end 150.519 83.59) (width 0.3048) (layer "F.Cu") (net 14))
 (via (at 150.519 83.59) (size 0.762) (drill 0.381) (layers "F.Cu" "B.Cu") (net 14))
 (segment (start 156.9466 84.201) (end 156.5727 84.201) (width 0.3048) (layer "B.Cu") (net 14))
 (segment (start 157.988 84.201) (end 156.9466 84.201) (width 0.3048) (layer "B.Cu") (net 14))
 (segment (start 153.8564 83.2599) (end 153.5264 83.5899) (width 0.3048) (layer "B.Cu") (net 14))
 (segment (start 153.5264 83.5899) (end 150.519 83.5899) (width 0.3048) (layer "B.Cu") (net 14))
 (segment (start 150.519 83.5899) (end 150.519 83.59) (width 0.3048) (layer "B.Cu") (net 14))
 (segment (start 156.5727 84.201) (end 155.6316 83.2599) (width 0.3048) (layer "B.Cu") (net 14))
 (segment (start 155.6316 83.2599) (end 153.8564 83.2599) (width 0.3048) (layer "B.Cu") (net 14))
 (segment (start 152.019 86.114) (end 152.019 84.328) (width 0.3048) (layer "F.Cu") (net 12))
 (via (at 152.019 84.328) (size 0.762) (drill 0.381) (layers "F.Cu" "B.Cu") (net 12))
 (segment (start 152.019 84.328) (end 152.15 84.197) (width 0.3048) (layer "B.Cu") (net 12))
 (segment (start 154.0684 83.7428) (end 155.4316 83.7428) (width 0.3048) (layer "B.Cu") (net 12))
 (segment (start 156.5248 84.836) (end 157.988 84.836) (width 0.3048) (layer "B.Cu") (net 12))
 (segment (start 152.15 84.197) (end 153.6142 84.197) (width 0.3048) (layer "B.Cu") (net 12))
 (segment (start 155.4316 83.7428) (end 156.5248 84.836) (width 0.3048) (layer "B.Cu") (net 12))
 (segment (start 153.6142 84.197) (end 154.0684 83.7428) (width 0.3048) (layer "B.Cu") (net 12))
 (segment (start 153.5908 85.1076) (end 153.7597 84.9387) (width 0.3048) (layer "F.Cu") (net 10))
 (segment (start 153.519 85.1076) (end 153.5908 85.1076) (width 0.3048) (layer "F.Cu") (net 10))
 (segment (start 153.519 86.114) (end 153.519 85.1076) (width 0.3048) (layer "F.Cu") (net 10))
 (via (at 153.7597 84.9387) (size 0.762) (drill 0.381) (layers "F.Cu" "B.Cu") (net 10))
 (segment (start 156.9466 85.471) (end 156.3481 85.471) (width 0.3048) (layer "B.Cu") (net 10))
 (segment (start 157.988 85.471) (end 156.9466 85.471) (width 0.3048) (layer "B.Cu") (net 10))
 (segment (start 154.4727 84.2257) (end 153.7597 84.9387) (width 0.3048) (layer "B.Cu") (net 10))
 (segment (start 155.1028 84.2257) (end 154.4727 84.2257) (width 0.3048) (layer "B.Cu") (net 10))
 (segment (start 156.3481 85.471) (end 155.1028 84.2257) (width 0.3048) (layer "B.Cu") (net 10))
 (segment (start 155.019 85.1076) (end 154.9633 85.1076) (width 0.3048) (layer "F.Cu") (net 8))
 (segment (start 154.9633 85.1076) (end 154.793 84.9373) (width 0.3048) (layer "F.Cu") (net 8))
 (segment (start 155.019 86.114) (end 155.019 85.1076) (width 0.3048) (layer "F.Cu") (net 8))
 (via (at 154.793 84.9373) (size 0.762) (drill 0.381) (layers "F.Cu" "B.Cu") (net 8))
 (segment (start 157.988 86.106) (end 156.007 86.106) (width 0.3048) (layer "B.Cu") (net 8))
 (segment (start 154.8156 84.9147) (end 154.793 84.9373) (width 0.3048) (layer "B.Cu") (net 8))
 (segment (start 156.007 86.106) (end 154.8156 84.9147) (width 0.3048) (layer "B.Cu") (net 8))
 (segment (start 154.305 86.15) (end 154.269 86.114) (width 0.3048) (layer "F.Cu") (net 9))
 (segment (start 154.305 87.0458) (end 154.305 86.15) (width 0.3048) (layer "F.Cu") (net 9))
 (via (at 154.305 87.0458) (size 0.762) (drill 0.381) (layers "F.Cu" "B.Cu") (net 9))
 (segment (start 157.988 86.741) (end 154.61 86.741) (width 0.3048) (layer "B.Cu") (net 9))
 (segment (start 154.61 86.741) (end 154.305 87.0458) (width 0.3048) (layer "B.Cu") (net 9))
 (segment (start 151.269 87.1939) (end 151.3962 87.3211) (width 0.3048) (layer "F.Cu") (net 13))
 (segment (start 151.269 86.114) (end 151.269 87.1939) (width 0.3048) (layer "F.Cu") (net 13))
 (via (at 151.3962 87.3211) (size 0.762) (drill 0.381) (layers "F.Cu" "B.Cu") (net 13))
 (segment (start 151.3962 87.3211) (end 152.3879 88.3128) (width 0.3048) (layer "B.Cu") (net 13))
 (segment (start 155.4581 88.011) (end 157.988 88.011) (width 0.3048) (layer "B.Cu") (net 13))
 (segment (start 152.3879 88.3128) (end 155.1563 88.3128) (width 0.3048) (layer "B.Cu") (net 13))
 (segment (start 155.1563 88.3128) (end 155.4581 88.011) (width 0.3048) (layer "B.Cu") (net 13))
 (segment (start 146.087199 82.818801) (end 146.242 82.664) (width 0.508) (layer "F.Cu") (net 16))
 (segment (start 146.087199 86.643625) (end 146.087199 82.818801) (width 0.508) (layer "F.Cu") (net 16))
 (segment (start 146.242 82.664) (end 147.119 82.664) (width 0.508) (layer "F.Cu") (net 16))
 (segment (start 142.781 88.773) (end 143.957824 88.773) (width 0.508) (layer "F.Cu") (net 16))
 (segment (start 143.957824 88.773) (end 146.087199 86.643625) (width 0.508) (layer "F.Cu") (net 16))
 (segment (start 145.401388 82.534487) (end 145.405136 82.530739) (width 0.508) (layer "F.Cu") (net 17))
 (segment (start 145.405136 82.352067) (end 145.843203 81.914) (width 0.508) (layer "F.Cu") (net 17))
 (segment (start 144.039 87.503) (end 145.401388 86.140612) (width 0.508) (layer "F.Cu") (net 17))
 (segment (start 146.011 81.914) (end 147.119 81.914) (width 0.508) (layer "F.Cu") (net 17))
 (segment (start 145.405136 82.530739) (end 145.405136 82.352067) (width 0.508) (layer "F.Cu") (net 17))
 (segment (start 145.401388 86.140612) (end 145.401388 82.534487) (width 0.508) (layer "F.Cu") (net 17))
 (segment (start 142.781 87.503) (end 144.039 87.503) (width 0.508) (layer "F.Cu") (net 17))
 (segment (start 145.843203 81.914) (end 146.011 81.914) (width 0.508) (layer "F.Cu") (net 17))
 (segment (start 145.528422 81.164) (end 147.119 81.164) (width 0.508) (layer "F.Cu") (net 18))
 (segment (start 144.644578 85.627422) (end 144.644578 83.356547) (width 0.508) (layer "F.Cu") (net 18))
 (segment (start 144.039 86.233) (end 144.644578 85.627422) (width 0.508) (layer "F.Cu") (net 18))
 (segment (start 144.644578 83.356547) (end 144.648612 83.352513) (width 0.508) (layer "F.Cu") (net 18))
 (segment (start 144.648612 83.352513) (end 144.648612 82.04381) (width 0.508) (layer "F.Cu") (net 18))
 (segment (start 142.781 86.233) (end 144.039 86.233) (width 0.508) (layer "F.Cu") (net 18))
 (segment (start 144.648612 82.04381) (end 145.528422 81.164) (width 0.508) (layer "F.Cu") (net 18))
 (segment (start 143.338242 83.693) (end 143.962801 83.068441) (width 0.508) (layer "F.Cu") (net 19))
 (segment (start 146.011 80.414) (end 147.119 80.414) (width 0.508) (layer "F.Cu") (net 19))
 (segment (start 142.781 83.693) (end 143.338242 83.693) (width 0.508) (layer "F.Cu") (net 19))
 (segment (start 145.042516 80.414) (end 146.011 80.414) (width 0.508) (layer "F.Cu") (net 19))
 (segment (start 143.962801 81.493715) (end 145.042516 80.414) (width 0.508) (layer "F.Cu") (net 19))
 (segment (start 143.962801 83.068441) (end 143.962801 81.493715) (width 0.508) (layer "F.Cu") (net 19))
 (segment (start 152.769 86.114) (end 152.769 87.2863) (width 0.3048) (layer "F.Cu") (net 11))
 (via (at 152.769 87.2863) (size 0.762) (drill 0.381) (layers "F.Cu" "B.Cu") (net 11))
 (segment (start 155.1686 87.376) (end 157.988 87.376) (width 0.3048) (layer "B.Cu") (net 11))
 (segment (start 152.769 87.2863) (end 153.2523 87.7696) (width 0.3048) (layer "B.Cu") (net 11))
 (segment (start 154.775 87.7696) (end 155.1686 87.376) (width 0.3048) (layer "B.Cu") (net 11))
 (segment (start 153.2523 87.7696) (end 154.775 87.7696) (width 0.3048) (layer "B.Cu") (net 11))
 (segment (start 149.769 86.114) (end 149.769 87.3345) (width 0.3048) (layer "F.Cu") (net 15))
 (via (at 149.769 87.3345) (size 0.762) (drill 0.381) (layers "F.Cu" "B.Cu") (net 15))
 (segment (start 156.7812 88.8114) (end 156.9466 88.646) (width 0.3048) (layer "B.Cu") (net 15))
 (segment (start 157.988 88.646) (end 156.9466 88.646) (width 0.3048) (layer "B.Cu") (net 15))
 (segment (start 149.769 87.3345) (end 151.2459 88.8114) (width 0.3048) (layer "B.Cu") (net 15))
 (segment (start 151.2459 88.8114) (end 156.7812 88.8114) (width 0.3048) (layer "B.Cu") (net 15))
 (segment (start 155.811 78.164) (end 155.603827 78.371173) (width 0.508) (layer "F.Cu") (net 7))
 (segment (start 155.603827 78.371173) (end 155.603827 79.603008) (width 0.508) (layer "F.Cu") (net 7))
 (segment (start 155.603827 79.603008) (end 155.603827 80.141823) (width 0.508) (layer "F.Cu") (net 7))
 (segment (start 156.919 78.164) (end 155.811 78.164) (width 0.508) (layer "F.Cu") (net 7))
 (via (at 155.603827 80.141823) (size 0.762) (drill 0.381) (layers "F.Cu" "B.Cu") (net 7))
 (segment (start 155.603827 80.680638) (end 155.603827 80.141823) (width 0.508) (layer "B.Cu") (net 7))
 (segment (start 155.603827 80.800827) (end 155.603827 80.680638) (width 0.508) (layer "B.Cu") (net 7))
 (segment (start 155.956 81.153) (end 155.603827 80.800827) (width 0.508) (layer "B.Cu") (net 7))
 (segment (start 156.919 77.414) (end 155.25 77.414) (width 0.508) (layer "F.Cu") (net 6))
 (segment (start 153.541086 79.122914) (end 153.541086 79.587018) (width 0.508) (layer "F.Cu") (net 6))
 (segment (start 155.25 77.414) (end 153.541086 79.122914) (width 0.508) (layer "F.Cu") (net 6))
 (segment (start 153.541086 79.587018) (end 153.541086 80.125833) (width 0.508) (layer "F.Cu") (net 6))
 (via (at 153.541086 80.125833) (size 0.762) (drill 0.381) (layers "F.Cu" "B.Cu") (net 6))
 (segment (start 153.541086 81.151086) (end 153.541086 80.664648) (width 0.508) (layer "B.Cu") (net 6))
 (segment (start 153.543 81.153) (end 153.541086 81.151086) (width 0.508) (layer "B.Cu") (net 6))
 (segment (start 153.541086 80.664648) (end 153.541086 80.125833) (width 0.508) (layer "B.Cu") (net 6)))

